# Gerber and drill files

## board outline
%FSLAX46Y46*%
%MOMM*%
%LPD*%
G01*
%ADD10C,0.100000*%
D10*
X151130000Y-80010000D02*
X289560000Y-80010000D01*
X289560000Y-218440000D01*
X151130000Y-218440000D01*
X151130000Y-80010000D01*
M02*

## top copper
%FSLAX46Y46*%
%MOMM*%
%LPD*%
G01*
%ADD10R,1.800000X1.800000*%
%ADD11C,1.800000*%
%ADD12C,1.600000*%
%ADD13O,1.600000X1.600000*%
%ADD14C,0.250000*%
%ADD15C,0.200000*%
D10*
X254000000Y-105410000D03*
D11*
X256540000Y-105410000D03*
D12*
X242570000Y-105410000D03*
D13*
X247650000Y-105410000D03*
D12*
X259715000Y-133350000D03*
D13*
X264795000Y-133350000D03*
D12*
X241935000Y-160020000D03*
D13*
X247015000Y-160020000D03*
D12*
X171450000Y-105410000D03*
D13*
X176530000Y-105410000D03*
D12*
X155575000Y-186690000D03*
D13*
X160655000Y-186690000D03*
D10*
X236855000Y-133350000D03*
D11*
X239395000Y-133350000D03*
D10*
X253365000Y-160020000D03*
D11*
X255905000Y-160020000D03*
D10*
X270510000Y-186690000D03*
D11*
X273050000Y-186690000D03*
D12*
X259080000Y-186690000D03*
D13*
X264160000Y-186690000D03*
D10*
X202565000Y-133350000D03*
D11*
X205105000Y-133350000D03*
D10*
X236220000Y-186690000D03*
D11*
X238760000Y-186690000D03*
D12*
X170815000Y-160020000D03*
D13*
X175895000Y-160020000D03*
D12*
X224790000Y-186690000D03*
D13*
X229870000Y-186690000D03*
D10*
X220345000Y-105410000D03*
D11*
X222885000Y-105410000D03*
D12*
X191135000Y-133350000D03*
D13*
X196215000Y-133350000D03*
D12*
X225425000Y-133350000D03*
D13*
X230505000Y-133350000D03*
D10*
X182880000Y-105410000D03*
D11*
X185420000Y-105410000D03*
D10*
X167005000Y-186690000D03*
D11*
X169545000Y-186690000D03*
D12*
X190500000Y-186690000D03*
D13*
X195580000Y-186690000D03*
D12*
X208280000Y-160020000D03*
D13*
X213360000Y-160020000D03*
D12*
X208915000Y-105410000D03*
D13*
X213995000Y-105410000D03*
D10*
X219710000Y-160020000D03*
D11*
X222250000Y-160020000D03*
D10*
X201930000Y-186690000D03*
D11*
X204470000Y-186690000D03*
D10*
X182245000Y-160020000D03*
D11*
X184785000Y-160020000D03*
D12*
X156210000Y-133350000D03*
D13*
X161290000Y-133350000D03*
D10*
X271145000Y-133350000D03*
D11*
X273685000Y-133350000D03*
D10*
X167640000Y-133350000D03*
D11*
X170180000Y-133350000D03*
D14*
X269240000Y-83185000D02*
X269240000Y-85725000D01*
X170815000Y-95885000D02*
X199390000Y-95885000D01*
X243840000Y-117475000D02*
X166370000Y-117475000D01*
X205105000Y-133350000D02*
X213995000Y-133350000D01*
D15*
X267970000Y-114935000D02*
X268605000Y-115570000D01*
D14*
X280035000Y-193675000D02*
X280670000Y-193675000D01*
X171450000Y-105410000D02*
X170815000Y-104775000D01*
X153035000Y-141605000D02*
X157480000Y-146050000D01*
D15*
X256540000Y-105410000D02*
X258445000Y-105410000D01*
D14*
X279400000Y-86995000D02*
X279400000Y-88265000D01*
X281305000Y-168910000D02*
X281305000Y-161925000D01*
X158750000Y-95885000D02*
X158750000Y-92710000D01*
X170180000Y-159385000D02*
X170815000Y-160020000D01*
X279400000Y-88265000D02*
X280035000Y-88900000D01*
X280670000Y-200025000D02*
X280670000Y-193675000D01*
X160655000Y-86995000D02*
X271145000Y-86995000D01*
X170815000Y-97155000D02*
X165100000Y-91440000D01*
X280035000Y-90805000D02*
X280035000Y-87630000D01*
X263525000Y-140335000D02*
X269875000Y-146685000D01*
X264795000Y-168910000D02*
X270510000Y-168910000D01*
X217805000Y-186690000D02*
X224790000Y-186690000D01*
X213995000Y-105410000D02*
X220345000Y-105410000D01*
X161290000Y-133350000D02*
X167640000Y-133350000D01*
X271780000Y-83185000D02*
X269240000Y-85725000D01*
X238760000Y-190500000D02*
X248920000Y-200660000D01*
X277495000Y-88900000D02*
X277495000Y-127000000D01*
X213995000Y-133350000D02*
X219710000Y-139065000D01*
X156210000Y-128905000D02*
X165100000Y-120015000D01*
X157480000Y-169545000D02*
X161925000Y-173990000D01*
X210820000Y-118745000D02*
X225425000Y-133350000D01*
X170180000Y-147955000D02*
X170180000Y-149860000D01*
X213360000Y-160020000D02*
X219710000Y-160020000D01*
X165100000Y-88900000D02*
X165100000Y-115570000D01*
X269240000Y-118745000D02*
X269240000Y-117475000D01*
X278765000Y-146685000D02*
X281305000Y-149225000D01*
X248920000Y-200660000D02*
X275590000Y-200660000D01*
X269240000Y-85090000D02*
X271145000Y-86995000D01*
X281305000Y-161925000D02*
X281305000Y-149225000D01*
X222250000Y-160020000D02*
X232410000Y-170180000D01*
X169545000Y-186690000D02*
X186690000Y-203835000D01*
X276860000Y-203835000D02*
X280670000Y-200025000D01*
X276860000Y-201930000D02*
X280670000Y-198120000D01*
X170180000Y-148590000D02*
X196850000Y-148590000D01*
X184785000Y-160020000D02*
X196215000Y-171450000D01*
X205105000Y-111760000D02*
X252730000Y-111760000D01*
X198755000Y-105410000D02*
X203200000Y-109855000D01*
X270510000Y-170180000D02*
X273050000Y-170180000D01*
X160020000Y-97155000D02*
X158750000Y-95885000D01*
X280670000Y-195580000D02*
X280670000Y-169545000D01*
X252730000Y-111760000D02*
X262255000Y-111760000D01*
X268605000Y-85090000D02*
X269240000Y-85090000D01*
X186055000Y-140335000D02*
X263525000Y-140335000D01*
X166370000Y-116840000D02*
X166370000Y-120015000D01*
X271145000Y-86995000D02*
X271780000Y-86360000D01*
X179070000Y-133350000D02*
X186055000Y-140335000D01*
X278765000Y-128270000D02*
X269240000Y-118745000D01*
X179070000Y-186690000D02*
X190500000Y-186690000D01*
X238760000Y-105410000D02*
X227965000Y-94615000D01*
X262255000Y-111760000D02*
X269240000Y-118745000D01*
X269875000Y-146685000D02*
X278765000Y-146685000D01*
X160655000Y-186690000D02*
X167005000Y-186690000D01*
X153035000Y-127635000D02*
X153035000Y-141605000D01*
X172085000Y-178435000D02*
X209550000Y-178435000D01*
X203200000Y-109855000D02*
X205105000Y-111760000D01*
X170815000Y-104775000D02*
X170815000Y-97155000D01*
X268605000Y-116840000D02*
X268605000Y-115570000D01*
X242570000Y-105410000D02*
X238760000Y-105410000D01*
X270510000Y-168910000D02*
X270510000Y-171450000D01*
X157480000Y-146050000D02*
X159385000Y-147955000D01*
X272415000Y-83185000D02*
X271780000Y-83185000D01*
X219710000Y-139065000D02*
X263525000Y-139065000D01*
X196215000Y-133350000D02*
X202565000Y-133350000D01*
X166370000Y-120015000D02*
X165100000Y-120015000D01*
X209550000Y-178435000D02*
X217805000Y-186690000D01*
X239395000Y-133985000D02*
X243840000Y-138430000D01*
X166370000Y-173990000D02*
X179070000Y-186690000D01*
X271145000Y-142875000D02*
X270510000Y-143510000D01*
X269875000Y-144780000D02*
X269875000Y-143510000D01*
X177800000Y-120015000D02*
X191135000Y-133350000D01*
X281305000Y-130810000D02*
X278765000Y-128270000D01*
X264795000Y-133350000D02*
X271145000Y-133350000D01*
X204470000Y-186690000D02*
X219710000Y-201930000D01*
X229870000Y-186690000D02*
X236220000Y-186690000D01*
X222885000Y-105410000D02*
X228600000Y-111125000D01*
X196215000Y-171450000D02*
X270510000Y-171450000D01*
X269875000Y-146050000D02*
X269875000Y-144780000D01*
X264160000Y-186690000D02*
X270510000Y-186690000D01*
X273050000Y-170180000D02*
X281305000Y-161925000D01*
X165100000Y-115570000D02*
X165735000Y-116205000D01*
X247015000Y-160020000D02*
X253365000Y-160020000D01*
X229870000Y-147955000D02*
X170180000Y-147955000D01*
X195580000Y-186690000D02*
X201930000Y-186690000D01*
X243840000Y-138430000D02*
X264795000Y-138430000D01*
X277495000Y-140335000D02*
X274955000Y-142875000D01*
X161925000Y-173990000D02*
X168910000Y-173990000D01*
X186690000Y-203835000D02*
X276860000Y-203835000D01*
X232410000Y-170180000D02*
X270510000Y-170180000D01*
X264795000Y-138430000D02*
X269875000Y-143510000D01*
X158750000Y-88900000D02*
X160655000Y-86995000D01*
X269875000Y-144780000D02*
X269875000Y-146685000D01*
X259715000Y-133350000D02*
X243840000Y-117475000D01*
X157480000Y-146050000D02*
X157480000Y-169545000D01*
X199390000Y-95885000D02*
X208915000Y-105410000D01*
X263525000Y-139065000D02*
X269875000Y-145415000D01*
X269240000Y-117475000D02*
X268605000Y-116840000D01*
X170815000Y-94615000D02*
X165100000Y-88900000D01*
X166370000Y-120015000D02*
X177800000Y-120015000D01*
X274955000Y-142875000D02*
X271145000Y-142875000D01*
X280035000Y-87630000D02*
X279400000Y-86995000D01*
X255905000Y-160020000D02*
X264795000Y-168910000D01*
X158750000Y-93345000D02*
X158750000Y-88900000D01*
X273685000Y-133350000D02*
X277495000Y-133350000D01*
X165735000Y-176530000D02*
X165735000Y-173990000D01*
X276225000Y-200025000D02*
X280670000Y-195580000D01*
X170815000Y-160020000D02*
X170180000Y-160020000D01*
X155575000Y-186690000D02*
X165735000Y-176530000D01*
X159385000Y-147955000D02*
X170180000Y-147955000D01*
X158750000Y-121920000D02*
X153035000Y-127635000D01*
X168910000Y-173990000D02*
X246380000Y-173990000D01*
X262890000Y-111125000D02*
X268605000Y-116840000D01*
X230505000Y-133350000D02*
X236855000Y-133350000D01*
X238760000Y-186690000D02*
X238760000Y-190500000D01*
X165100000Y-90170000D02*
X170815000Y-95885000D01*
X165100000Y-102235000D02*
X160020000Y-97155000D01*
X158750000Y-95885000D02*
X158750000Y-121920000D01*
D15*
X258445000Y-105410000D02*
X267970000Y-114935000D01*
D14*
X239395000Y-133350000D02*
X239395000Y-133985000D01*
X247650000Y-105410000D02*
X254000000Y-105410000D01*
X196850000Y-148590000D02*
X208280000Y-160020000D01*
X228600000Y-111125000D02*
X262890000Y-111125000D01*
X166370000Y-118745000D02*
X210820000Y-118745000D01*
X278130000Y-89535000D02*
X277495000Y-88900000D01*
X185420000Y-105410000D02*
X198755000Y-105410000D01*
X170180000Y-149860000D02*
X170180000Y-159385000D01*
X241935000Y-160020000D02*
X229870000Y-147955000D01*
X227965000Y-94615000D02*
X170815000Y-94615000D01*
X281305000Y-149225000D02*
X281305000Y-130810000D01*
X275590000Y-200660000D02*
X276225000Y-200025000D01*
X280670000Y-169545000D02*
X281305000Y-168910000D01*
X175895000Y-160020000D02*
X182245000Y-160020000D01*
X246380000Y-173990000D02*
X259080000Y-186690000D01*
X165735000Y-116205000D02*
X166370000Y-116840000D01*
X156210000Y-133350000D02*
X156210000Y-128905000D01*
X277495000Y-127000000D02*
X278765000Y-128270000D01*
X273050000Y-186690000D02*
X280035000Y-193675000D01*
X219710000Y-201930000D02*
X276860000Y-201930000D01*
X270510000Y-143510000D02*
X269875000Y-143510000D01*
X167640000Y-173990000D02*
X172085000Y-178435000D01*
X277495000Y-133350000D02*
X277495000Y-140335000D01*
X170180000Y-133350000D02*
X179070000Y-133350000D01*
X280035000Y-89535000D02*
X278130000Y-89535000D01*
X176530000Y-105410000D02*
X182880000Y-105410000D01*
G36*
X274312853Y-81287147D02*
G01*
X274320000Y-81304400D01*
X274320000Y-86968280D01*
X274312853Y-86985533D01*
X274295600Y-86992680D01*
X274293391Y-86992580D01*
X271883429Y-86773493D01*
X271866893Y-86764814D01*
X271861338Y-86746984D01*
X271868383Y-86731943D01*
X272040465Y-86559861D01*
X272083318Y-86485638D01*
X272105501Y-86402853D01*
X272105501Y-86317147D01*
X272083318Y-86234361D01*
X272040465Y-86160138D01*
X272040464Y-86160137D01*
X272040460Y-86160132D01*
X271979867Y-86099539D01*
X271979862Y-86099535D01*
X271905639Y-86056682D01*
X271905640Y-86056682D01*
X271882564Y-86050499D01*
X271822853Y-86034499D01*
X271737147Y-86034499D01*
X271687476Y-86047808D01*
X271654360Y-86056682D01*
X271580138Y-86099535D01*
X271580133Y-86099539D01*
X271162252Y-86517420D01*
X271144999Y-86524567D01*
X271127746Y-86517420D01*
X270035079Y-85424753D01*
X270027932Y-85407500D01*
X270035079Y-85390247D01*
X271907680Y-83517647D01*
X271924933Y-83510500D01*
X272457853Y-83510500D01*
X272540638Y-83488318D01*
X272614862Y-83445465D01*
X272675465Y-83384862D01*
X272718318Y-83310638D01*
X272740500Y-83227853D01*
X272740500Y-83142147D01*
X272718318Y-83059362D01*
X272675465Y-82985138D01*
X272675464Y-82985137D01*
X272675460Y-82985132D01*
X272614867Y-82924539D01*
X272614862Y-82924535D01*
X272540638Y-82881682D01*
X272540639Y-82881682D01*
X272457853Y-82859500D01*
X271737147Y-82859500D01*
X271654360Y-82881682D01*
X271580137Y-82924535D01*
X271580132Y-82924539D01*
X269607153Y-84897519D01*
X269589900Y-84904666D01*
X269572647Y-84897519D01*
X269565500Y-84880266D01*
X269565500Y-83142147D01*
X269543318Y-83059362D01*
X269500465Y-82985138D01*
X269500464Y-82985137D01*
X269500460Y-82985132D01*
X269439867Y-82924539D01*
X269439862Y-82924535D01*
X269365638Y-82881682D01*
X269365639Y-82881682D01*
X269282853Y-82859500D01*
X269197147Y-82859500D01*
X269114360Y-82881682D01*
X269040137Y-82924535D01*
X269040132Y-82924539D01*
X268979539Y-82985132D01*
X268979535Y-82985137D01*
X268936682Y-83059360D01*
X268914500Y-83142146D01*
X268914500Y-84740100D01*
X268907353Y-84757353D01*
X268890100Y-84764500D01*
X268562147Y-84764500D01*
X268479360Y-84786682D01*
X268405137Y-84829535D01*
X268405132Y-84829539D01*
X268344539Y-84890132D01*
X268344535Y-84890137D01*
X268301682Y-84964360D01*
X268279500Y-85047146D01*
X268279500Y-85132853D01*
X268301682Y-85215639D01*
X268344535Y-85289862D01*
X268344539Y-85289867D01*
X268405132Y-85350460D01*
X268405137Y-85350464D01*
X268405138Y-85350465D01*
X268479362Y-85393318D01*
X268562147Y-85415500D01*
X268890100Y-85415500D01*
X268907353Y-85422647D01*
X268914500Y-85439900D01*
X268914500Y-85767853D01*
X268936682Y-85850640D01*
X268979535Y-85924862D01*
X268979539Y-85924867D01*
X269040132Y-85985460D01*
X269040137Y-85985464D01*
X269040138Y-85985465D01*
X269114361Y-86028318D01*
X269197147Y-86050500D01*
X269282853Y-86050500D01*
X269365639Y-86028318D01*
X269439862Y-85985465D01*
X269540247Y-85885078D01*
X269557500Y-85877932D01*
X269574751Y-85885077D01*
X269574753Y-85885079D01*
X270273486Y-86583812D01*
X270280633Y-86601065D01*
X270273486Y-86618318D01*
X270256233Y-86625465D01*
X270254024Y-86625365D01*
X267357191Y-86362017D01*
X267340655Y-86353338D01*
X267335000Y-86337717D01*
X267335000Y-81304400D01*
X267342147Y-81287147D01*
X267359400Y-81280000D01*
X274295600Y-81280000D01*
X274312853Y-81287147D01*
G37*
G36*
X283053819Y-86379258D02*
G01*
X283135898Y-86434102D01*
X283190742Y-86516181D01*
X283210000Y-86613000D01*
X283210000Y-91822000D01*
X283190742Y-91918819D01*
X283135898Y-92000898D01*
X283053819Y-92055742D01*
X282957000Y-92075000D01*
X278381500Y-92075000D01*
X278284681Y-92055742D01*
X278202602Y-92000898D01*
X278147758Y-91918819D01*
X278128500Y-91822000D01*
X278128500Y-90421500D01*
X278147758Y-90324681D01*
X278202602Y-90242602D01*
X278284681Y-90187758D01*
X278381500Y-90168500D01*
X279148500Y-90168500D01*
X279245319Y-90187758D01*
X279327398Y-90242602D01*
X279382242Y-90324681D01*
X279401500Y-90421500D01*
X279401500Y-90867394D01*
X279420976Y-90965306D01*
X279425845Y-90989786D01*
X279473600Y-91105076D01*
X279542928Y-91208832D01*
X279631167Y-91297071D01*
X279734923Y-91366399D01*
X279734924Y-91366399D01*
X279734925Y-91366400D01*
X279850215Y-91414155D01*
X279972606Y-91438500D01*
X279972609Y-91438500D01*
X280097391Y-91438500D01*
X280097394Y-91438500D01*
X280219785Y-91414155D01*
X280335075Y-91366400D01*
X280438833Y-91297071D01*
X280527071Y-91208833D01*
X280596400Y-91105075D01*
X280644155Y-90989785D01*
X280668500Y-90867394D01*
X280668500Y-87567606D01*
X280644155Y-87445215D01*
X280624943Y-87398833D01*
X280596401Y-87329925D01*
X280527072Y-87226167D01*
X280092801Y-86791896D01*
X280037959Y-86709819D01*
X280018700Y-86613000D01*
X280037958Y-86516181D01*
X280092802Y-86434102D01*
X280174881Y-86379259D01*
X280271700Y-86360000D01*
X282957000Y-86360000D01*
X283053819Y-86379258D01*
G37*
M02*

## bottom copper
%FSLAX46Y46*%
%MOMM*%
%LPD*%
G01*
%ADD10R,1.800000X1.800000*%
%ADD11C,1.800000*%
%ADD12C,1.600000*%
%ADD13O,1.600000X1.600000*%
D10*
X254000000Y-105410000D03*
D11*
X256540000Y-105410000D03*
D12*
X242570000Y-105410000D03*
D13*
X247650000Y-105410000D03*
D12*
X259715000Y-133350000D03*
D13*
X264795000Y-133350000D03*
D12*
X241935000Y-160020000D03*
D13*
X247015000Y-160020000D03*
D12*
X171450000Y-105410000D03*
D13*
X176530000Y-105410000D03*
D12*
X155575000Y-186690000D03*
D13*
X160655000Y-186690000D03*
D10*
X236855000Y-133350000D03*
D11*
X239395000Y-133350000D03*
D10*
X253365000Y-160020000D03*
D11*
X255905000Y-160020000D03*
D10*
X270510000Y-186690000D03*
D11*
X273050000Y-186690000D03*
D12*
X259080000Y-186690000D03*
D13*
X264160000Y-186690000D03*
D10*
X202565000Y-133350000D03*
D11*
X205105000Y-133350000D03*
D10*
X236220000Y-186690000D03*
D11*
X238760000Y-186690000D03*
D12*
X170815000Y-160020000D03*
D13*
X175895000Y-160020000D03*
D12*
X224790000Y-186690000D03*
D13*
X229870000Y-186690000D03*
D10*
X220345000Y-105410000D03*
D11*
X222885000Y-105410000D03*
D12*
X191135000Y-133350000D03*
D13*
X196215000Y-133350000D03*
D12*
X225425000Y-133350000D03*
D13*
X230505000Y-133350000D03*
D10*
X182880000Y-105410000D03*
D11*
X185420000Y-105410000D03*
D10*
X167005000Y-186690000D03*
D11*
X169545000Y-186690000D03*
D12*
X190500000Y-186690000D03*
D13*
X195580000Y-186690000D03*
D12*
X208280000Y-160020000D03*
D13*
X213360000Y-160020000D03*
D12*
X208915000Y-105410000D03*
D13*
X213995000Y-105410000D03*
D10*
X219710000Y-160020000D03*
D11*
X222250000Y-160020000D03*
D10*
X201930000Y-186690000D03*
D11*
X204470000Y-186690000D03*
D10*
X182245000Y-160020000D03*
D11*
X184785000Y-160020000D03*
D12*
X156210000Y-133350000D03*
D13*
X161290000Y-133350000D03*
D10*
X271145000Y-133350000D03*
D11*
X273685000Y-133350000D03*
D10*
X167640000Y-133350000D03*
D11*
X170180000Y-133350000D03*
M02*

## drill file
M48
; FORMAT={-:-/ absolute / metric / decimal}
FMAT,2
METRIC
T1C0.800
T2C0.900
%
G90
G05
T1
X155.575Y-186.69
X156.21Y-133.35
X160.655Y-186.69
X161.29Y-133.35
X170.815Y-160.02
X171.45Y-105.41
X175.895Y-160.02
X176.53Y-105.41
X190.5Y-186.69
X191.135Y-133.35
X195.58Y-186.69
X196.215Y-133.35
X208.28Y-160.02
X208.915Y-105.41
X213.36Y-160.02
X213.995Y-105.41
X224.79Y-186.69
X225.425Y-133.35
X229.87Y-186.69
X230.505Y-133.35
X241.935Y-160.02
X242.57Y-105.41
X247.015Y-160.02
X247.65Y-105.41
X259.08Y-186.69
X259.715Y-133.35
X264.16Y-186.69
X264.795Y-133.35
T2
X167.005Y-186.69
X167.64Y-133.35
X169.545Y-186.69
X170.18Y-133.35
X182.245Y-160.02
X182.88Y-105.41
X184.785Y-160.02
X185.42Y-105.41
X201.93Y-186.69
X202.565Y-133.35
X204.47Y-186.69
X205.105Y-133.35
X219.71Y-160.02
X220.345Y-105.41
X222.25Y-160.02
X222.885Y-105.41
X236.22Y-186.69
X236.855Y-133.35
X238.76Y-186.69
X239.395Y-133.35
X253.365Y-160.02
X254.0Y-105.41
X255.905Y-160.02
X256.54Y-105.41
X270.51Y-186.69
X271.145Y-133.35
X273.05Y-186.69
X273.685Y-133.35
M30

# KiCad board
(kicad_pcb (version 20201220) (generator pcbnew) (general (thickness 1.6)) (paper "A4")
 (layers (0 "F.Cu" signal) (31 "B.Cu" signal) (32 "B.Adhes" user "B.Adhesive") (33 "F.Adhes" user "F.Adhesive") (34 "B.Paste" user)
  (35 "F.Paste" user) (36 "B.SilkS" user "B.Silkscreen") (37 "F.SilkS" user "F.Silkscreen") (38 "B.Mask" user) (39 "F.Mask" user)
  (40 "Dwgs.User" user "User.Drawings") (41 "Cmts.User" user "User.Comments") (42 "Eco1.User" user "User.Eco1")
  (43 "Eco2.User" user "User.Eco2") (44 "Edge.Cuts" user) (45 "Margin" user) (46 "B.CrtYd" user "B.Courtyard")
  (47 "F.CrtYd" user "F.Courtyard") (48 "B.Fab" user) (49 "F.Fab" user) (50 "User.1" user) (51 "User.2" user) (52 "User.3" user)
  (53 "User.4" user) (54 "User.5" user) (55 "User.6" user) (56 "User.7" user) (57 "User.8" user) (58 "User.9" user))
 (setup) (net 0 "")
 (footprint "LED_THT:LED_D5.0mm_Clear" (layer "F.Cu") (at 254 105.41)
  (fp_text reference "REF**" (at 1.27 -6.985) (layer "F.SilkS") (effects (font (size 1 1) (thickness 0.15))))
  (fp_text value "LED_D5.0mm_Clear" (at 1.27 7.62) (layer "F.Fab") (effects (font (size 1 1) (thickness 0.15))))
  (pad "1" thru_hole rect (at 0 0) (size 1.8 1.8) (drill 0.9) (layers *.Cu *.Mask))
  (pad "2" thru_hole circle (at 2.54 0) (size 1.8 1.8) (drill 0.9) (layers *.Cu *.Mask)))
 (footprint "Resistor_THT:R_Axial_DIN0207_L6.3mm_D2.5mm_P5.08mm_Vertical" (layer "F.Cu") (at 242.57 105.41)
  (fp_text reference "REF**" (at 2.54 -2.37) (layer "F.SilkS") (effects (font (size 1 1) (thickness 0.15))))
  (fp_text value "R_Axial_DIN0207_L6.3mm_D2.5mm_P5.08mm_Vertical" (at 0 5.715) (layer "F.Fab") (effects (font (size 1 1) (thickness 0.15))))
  (pad "1" thru_hole circle (at 0 0) (size 1.6 1.6) (drill 0.8) (layers *.Cu *.Mask))
  (pad "2" thru_hole oval (at 5.08 0) (size 1.6 1.6) (drill 0.8) (layers *.Cu *.Mask)))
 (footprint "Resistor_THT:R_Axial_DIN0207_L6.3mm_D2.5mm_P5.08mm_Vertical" (layer "F.Cu") (at 259.715 133.35)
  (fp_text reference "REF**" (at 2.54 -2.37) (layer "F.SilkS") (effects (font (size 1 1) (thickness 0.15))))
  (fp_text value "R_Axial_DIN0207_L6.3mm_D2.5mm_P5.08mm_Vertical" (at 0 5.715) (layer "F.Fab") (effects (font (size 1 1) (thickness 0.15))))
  (pad "1" thru_hole circle (at 0 0) (size 1.6 1.6) (drill 0.8) (layers *.Cu *.Mask))
  (pad "2" thru_hole oval (at 5.08 0) (size 1.6 1.6) (drill 0.8) (layers *.Cu *.Mask)))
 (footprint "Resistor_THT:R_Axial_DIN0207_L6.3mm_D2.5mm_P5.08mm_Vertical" (layer "F.Cu") (at 241.935 160.02)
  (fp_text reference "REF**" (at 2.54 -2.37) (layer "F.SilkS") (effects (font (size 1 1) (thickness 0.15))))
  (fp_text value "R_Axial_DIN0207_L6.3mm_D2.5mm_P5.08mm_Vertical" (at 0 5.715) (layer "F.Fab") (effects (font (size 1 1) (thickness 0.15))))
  (pad "1" thru_hole circle (at 0 0) (size 1.6 1.6) (drill 0.8) (layers *.Cu *.Mask))
  (pad "2" thru_hole oval (at 5.08 0) (size 1.6 1.6) (drill 0.8) (layers *.Cu *.Mask)))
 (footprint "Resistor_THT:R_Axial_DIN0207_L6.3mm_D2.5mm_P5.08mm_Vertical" (layer "F.Cu") (at 171.45 105.41)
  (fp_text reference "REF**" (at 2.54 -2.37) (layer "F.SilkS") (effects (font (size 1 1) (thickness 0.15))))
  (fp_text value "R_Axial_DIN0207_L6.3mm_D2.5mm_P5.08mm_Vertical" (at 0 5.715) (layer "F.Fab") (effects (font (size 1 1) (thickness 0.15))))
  (pad "1" thru_hole circle (at 0 0) (size 1.6 1.6) (drill 0.8) (layers *.Cu *.Mask))
  (pad "2" thru_hole oval (at 5.08 0) (size 1.6 1.6) (drill 0.8) (layers *.Cu *.Mask)))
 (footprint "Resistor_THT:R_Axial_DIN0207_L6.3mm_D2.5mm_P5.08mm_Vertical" (layer "F.Cu") (at 155.575 186.69)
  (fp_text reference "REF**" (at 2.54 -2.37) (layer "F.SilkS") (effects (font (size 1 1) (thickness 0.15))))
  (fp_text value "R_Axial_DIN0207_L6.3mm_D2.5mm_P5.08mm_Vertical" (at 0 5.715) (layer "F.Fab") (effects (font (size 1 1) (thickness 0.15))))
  (pad "1" thru_hole circle (at 0 0) (size 1.6 1.6) (drill 0.8) (layers *.Cu *.Mask))
  (pad "2" thru_hole oval (at 5.08 0) (size 1.6 1.6) (drill 0.8) (layers *.Cu *.Mask)))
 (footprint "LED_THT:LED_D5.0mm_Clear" (layer "F.Cu") (at 236.855 133.35)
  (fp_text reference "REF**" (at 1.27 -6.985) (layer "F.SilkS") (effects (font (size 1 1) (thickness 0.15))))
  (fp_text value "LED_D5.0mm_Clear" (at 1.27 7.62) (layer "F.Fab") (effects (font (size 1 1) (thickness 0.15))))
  (pad "1" thru_hole rect (at 0 0) (size 1.8 1.8) (drill 0.9) (layers *.Cu *.Mask))
  (pad "2" thru_hole circle (at 2.54 0) (size 1.8 1.8) (drill 0.9) (layers *.Cu *.Mask)))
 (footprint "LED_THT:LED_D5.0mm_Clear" (layer "F.Cu") (at 253.365 160.02)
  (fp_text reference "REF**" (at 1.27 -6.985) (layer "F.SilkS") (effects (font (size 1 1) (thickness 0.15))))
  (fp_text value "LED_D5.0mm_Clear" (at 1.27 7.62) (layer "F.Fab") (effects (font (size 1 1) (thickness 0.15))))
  (pad "1" thru_hole rect (at 0 0) (size 1.8 1.8) (drill 0.9) (layers *.Cu *.Mask))
  (pad "2" thru_hole circle (at 2.54 0) (size 1.8 1.8) (drill 0.9) (layers *.Cu *.Mask)))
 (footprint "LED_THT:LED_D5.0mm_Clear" (layer "F.Cu") (at 270.51 186.69)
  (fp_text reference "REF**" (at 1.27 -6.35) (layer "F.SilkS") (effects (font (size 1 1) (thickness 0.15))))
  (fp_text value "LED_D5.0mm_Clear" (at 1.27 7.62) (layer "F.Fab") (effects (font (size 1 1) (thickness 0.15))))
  (pad "1" thru_hole rect (at 0 0) (size 1.8 1.8) (drill 0.9) (layers *.Cu *.Mask))
  (pad "2" thru_hole circle (at 2.54 0) (size 1.8 1.8) (drill 0.9) (layers *.Cu *.Mask)))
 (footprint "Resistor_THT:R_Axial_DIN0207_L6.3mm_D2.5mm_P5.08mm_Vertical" (layer "F.Cu") (at 259.08 186.69)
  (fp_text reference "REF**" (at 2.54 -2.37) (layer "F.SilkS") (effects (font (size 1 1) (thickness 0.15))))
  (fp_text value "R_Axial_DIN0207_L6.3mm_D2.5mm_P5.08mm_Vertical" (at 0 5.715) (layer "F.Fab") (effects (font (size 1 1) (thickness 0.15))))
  (pad "1" thru_hole circle (at 0 0) (size 1.6 1.6) (drill 0.8) (layers *.Cu *.Mask))
  (pad "2" thru_hole oval (at 5.08 0) (size 1.6 1.6) (drill 0.8) (layers *.Cu *.Mask)))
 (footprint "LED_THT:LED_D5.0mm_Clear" (layer "F.Cu") (at 202.565 133.35)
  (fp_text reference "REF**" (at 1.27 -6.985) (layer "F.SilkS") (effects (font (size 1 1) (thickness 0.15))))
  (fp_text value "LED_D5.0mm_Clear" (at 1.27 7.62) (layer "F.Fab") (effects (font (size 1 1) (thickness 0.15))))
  (pad "1" thru_hole rect (at 0 0) (size 1.8 1.8) (drill 0.9) (layers *.Cu *.Mask))
  (pad "2" thru_hole circle (at 2.54 0) (size 1.8 1.8) (drill 0.9) (layers *.Cu *.Mask)))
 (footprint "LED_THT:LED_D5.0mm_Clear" (layer "F.Cu") (at 236.22 186.69)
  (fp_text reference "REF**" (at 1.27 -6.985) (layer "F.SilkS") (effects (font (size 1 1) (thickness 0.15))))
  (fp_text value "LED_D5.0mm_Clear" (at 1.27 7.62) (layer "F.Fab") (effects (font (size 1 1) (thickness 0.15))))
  (pad "1" thru_hole rect (at 0 0) (size 1.8 1.8) (drill 0.9) (layers *.Cu *.Mask))
  (pad "2" thru_hole circle (at 2.54 0) (size 1.8 1.8) (drill 0.9) (layers *.Cu *.Mask)))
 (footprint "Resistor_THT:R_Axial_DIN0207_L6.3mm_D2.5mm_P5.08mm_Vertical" (layer "F.Cu") (at 170.815 160.02)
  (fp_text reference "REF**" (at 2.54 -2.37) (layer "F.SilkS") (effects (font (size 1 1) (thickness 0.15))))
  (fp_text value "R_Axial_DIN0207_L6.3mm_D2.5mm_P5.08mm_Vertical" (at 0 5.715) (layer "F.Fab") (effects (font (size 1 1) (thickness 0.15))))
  (pad "1" thru_hole circle (at 0 0) (size 1.6 1.6) (drill 0.8) (layers *.Cu *.Mask))
  (pad "2" thru_hole oval (at 5.08 0) (size 1.6 1.6) (drill 0.8) (layers *.Cu *.Mask)))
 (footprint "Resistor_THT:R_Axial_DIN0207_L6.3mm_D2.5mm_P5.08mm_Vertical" (layer "F.Cu") (at 224.79 186.69)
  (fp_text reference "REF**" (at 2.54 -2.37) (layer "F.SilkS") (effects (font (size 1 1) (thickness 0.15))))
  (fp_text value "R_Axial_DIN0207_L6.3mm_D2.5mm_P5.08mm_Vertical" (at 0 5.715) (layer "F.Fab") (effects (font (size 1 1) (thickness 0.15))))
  (pad "1" thru_hole circle (at 0 0) (size 1.6 1.6) (drill 0.8) (layers *.Cu *.Mask))
  (pad "2" thru_hole oval (at 5.08 0) (size 1.6 1.6) (drill 0.8) (layers *.Cu *.Mask)))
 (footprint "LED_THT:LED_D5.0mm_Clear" (layer "F.Cu") (at 220.345 105.41)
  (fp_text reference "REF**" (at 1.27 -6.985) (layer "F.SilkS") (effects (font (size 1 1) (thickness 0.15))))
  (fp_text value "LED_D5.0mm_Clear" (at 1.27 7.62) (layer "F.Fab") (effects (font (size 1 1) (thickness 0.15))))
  (pad "1" thru_hole rect (at 0 0) (size 1.8 1.8) (drill 0.9) (layers *.Cu *.Mask))
  (pad "2" thru_hole circle (at 2.54 0) (size 1.8 1.8) (drill 0.9) (layers *.Cu *.Mask)))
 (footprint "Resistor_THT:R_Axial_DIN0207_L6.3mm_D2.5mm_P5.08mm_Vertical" (layer "F.Cu") (at 191.135 133.35)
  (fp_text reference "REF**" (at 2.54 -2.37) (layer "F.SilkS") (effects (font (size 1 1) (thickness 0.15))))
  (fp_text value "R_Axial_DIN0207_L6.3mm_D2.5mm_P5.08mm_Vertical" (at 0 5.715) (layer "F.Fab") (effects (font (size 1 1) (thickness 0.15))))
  (pad "1" thru_hole circle (at 0 0) (size 1.6 1.6) (drill 0.8) (layers *.Cu *.Mask))
  (pad "2" thru_hole oval (at 5.08 0) (size 1.6 1.6) (drill 0.8) (layers *.Cu *.Mask)))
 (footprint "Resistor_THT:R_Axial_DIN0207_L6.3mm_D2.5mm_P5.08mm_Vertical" (layer "F.Cu") (at 225.425 133.35)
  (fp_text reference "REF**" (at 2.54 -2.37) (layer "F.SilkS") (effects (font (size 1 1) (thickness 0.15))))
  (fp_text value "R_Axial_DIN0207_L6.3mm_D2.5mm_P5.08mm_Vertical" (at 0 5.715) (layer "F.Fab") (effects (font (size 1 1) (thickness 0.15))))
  (pad "1" thru_hole circle (at 0 0) (size 1.6 1.6) (drill 0.8) (layers *.Cu *.Mask))
  (pad "2" thru_hole oval (at 5.08 0) (size 1.6 1.6) (drill 0.8) (layers *.Cu *.Mask)))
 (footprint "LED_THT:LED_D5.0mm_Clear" (layer "F.Cu") (at 182.88 105.41)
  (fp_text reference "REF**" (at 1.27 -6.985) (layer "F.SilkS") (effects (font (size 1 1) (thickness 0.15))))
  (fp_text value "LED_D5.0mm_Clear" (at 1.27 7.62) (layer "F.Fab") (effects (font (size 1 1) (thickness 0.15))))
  (pad "1" thru_hole rect (at 0 0) (size 1.8 1.8) (drill 0.9) (layers *.Cu *.Mask))
  (pad "2" thru_hole circle (at 2.54 0) (size 1.8 1.8) (drill 0.9) (layers *.Cu *.Mask)))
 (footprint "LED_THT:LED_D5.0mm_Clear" (layer "F.Cu") (at 167.005 186.69)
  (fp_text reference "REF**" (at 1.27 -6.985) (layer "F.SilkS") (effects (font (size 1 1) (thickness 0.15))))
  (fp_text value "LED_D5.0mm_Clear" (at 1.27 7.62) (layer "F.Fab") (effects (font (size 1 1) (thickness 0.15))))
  (pad "1" thru_hole rect (at 0 0) (size 1.8 1.8) (drill 0.9) (layers *.Cu *.Mask))
  (pad "2" thru_hole circle (at 2.54 0) (size 1.8 1.8) (drill 0.9) (layers *.Cu *.Mask)))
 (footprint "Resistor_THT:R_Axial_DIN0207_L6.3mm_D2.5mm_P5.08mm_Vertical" (layer "F.Cu") (at 190.5 186.69)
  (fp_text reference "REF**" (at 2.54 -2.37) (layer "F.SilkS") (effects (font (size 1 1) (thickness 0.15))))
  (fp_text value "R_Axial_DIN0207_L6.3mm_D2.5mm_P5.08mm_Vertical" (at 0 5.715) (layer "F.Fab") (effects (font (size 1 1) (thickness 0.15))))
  (pad "1" thru_hole circle (at 0 0) (size 1.6 1.6) (drill 0.8) (layers *.Cu *.Mask))
  (pad "2" thru_hole oval (at 5.08 0) (size 1.6 1.6) (drill 0.8) (layers *.Cu *.Mask)))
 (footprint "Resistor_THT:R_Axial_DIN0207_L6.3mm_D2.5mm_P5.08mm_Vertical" (layer "F.Cu") (at 208.28 160.02)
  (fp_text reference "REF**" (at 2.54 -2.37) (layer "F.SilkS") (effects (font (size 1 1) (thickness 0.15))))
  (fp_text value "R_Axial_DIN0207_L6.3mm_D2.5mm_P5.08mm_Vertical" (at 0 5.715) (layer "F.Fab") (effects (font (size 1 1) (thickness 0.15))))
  (pad "1" thru_hole circle (at 0 0) (size 1.6 1.6) (drill 0.8) (layers *.Cu *.Mask))
  (pad "2" thru_hole oval (at 5.08 0) (size 1.6 1.6) (drill 0.8) (layers *.Cu *.Mask)))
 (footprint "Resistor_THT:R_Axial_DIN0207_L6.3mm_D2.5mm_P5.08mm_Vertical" (layer "F.Cu") (at 208.915 105.41)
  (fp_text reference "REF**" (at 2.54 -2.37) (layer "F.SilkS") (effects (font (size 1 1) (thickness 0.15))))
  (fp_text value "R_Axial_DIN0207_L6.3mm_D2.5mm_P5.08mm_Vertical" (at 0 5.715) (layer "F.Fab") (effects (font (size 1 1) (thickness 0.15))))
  (pad "1" thru_hole circle (at 0 0) (size 1.6 1.6) (drill 0.8) (layers *.Cu *.Mask))
  (pad "2" thru_hole oval (at 5.08 0) (size 1.6 1.6) (drill 0.8) (layers *.Cu *.Mask)))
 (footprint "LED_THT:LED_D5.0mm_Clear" (layer "F.Cu") (at 219.71 160.02)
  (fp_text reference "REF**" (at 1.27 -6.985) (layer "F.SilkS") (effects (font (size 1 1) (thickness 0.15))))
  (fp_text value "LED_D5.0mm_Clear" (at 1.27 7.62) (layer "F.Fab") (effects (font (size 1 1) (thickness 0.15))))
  (pad "1" thru_hole rect (at 0 0) (size 1.8 1.8) (drill 0.9) (layers *.Cu *.Mask))
  (pad "2" thru_hole circle (at 2.54 0) (size 1.8 1.8) (drill 0.9) (layers *.Cu *.Mask)))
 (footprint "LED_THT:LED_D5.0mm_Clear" (layer "F.Cu") (at 201.93 186.69)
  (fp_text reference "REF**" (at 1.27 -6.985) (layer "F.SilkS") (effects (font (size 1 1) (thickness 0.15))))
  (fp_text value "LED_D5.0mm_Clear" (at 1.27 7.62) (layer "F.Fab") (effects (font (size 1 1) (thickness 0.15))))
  (pad "1" thru_hole rect (at 0 0) (size 1.8 1.8) (drill 0.9) (layers *.Cu *.Mask))
  (pad "2" thru_hole circle (at 2.54 0) (size 1.8 1.8) (drill 0.9) (layers *.Cu *.Mask)))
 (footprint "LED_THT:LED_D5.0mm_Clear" (layer "F.Cu") (at 182.245 160.02)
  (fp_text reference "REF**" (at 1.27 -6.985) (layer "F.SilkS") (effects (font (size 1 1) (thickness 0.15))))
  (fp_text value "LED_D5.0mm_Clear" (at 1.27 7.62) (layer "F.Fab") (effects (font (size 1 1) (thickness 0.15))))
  (pad "1" thru_hole rect (at 0 0) (size 1.8 1.8) (drill 0.9) (layers *.Cu *.Mask))
  (pad "2" thru_hole circle (at 2.54 0) (size 1.8 1.8) (drill 0.9) (layers *.Cu *.Mask)))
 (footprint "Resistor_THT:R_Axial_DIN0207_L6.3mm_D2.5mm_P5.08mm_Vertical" (layer "F.Cu") (at 156.21 133.35)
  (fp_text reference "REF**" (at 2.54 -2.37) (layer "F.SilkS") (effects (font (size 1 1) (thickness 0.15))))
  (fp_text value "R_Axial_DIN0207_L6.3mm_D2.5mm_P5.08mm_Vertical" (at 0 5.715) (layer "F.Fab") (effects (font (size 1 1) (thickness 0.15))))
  (pad "1" thru_hole circle (at 0 0) (size 1.6 1.6) (drill 0.8) (layers *.Cu *.Mask))
  (pad "2" thru_hole oval (at 5.08 0) (size 1.6 1.6) (drill 0.8) (layers *.Cu *.Mask)))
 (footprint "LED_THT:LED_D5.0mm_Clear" (layer "F.Cu") (at 271.145 133.35)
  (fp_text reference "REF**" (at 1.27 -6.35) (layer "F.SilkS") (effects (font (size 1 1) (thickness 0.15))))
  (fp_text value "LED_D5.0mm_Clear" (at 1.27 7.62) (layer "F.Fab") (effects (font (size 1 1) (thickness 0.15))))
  (pad "1" thru_hole rect (at 0 0) (size 1.8 1.8) (drill 0.9) (layers *.Cu *.Mask))
  (pad "2" thru_hole circle (at 2.54 0) (size 1.8 1.8) (drill 0.9) (layers *.Cu *.Mask)))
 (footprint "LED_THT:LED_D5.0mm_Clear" (layer "F.Cu") (at 167.64 133.35)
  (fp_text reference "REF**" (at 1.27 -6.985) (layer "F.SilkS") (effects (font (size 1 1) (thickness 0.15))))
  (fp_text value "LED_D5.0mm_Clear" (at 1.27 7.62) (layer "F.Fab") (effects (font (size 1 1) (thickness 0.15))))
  (pad "1" thru_hole rect (at 0 0) (size 1.8 1.8) (drill 0.9) (layers *.Cu *.Mask))
  (pad "2" thru_hole circle (at 2.54 0) (size 1.8 1.8) (drill 0.9) (layers *.Cu *.Mask)))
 (gr_rect (start 151.13 80.01) (end 289.56 218.44) (layer "Edge.Cuts") (width 0.1) (fill none))
 (segment (start 269.24 83.185) (end 269.24 85.725) (width 0.25) (layer "F.Cu") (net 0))
 (segment (start 170.815 95.885) (end 199.39 95.885) (width 0.25) (layer "F.Cu") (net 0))
 (segment (start 243.84 117.475) (end 166.37 117.475) (width 0.25) (layer "F.Cu") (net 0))
 (segment (start 205.105 133.35) (end 213.995 133.35) (width 0.25) (layer "F.Cu") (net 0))
 (segment (start 267.97 114.935) (end 268.605 115.57) (width 0.2) (layer "F.Cu") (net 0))
 (segment (start 280.035 193.675) (end 280.67 193.675) (width 0.25) (layer "F.Cu") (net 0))
 (segment (start 171.45 105.41) (end 170.815 104.775) (width 0.25) (layer "F.Cu") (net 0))
 (segment (start 153.035 141.605) (end 157.48 146.05) (width 0.25) (layer "F.Cu") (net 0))
 (segment (start 256.54 105.41) (end 258.445 105.41) (width 0.2) (layer "F.Cu") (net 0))
 (segment (start 279.4 86.995) (end 279.4 88.265) (width 0.25) (layer "F.Cu") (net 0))
 (segment (start 281.305 168.91) (end 281.305 161.925) (width 0.25) (layer "F.Cu") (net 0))
 (segment (start 158.75 95.885) (end 158.75 92.71) (width 0.25) (layer "F.Cu") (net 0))
 (segment (start 170.18 159.385) (end 170.815 160.02) (width 0.25) (layer "F.Cu") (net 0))
 (segment (start 279.4 88.265) (end 280.035 88.9) (width 0.25) (layer "F.Cu") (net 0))
 (segment (start 280.67 200.025) (end 280.67 193.675) (width 0.25) (layer "F.Cu") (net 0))
 (segment (start 160.655 86.995) (end 271.145 86.995) (width 0.25) (layer "F.Cu") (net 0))
 (segment (start 170.815 97.155) (end 165.1 91.44) (width 0.25) (layer "F.Cu") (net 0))
 (segment (start 280.035 90.805) (end 280.035 87.63) (width 0.25) (layer "F.Cu") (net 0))
 (segment (start 263.525 140.335) (end 269.875 146.685) (width 0.25) (layer "F.Cu") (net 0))
 (segment (start 264.795 168.91) (end 270.51 168.91) (width 0.25) (layer "F.Cu") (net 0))
 (segment (start 217.805 186.69) (end 224.79 186.69) (width 0.25) (layer "F.Cu") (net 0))
 (segment (start 213.995 105.41) (end 220.345 105.41) (width 0.25) (layer "F.Cu") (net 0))
 (segment (start 161.29 133.35) (end 167.64 133.35) (width 0.25) (layer "F.Cu") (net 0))
 (segment (start 271.78 83.185) (end 269.24 85.725) (width 0.25) (layer "F.Cu") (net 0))
 (segment (start 238.76 190.5) (end 248.92 200.66) (width 0.25) (layer "F.Cu") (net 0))
 (segment (start 277.495 88.9) (end 277.495 127) (width 0.25) (layer "F.Cu") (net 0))
 (segment (start 213.995 133.35) (end 219.71 139.065) (width 0.25) (layer "F.Cu") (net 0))
 (segment (start 156.21 128.905) (end 165.1 120.015) (width 0.25) (layer "F.Cu") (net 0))
 (segment (start 157.48 169.545) (end 161.925 173.99) (width 0.25) (layer "F.Cu") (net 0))
 (segment (start 210.82 118.745) (end 225.425 133.35) (width 0.25) (layer "F.Cu") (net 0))
 (segment (start 170.18 147.955) (end 170.18 149.86) (width 0.25) (layer "F.Cu") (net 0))
 (segment (start 213.36 160.02) (end 219.71 160.02) (width 0.25) (layer "F.Cu") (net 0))
 (segment (start 165.1 88.9) (end 165.1 115.57) (width 0.25) (layer "F.Cu") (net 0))
 (segment (start 269.24 118.745) (end 269.24 117.475) (width 0.25) (layer "F.Cu") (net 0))
 (segment (start 278.765 146.685) (end 281.305 149.225) (width 0.25) (layer "F.Cu") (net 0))
 (segment (start 248.92 200.66) (end 275.59 200.66) (width 0.25) (layer "F.Cu") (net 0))
 (segment (start 269.24 85.09) (end 271.145 86.995) (width 0.25) (layer "F.Cu") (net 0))
 (segment (start 281.305 161.925) (end 281.305 149.225) (width 0.25) (layer "F.Cu") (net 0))
 (segment (start 222.25 160.02) (end 232.41 170.18) (width 0.25) (layer "F.Cu") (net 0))
 (segment (start 169.545 186.69) (end 186.69 203.835) (width 0.25) (layer "F.Cu") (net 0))
 (segment (start 276.86 203.835) (end 280.67 200.025) (width 0.25) (layer "F.Cu") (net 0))
 (segment (start 276.86 201.93) (end 280.67 198.12) (width 0.25) (layer "F.Cu") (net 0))
 (segment (start 170.18 148.59) (end 196.85 148.59) (width 0.25) (layer "F.Cu") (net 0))
 (segment (start 184.785 160.02) (end 196.215 171.45) (width 0.25) (layer "F.Cu") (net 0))
 (segment (start 205.105 111.76) (end 252.73 111.76) (width 0.25) (layer "F.Cu") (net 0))
 (segment (start 198.755 105.41) (end 203.2 109.855) (width 0.25) (layer "F.Cu") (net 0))
 (segment (start 270.51 170.18) (end 273.05 170.18) (width 0.25) (layer "F.Cu") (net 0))
 (segment (start 160.02 97.155) (end 158.75 95.885) (width 0.25) (layer "F.Cu") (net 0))
 (segment (start 280.67 195.58) (end 280.67 169.545) (width 0.25) (layer "F.Cu") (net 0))
 (segment (start 252.73 111.76) (end 262.255 111.76) (width 0.25) (layer "F.Cu") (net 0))
 (segment (start 268.605 85.09) (end 269.24 85.09) (width 0.25) (layer "F.Cu") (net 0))
 (segment (start 186.055 140.335) (end 263.525 140.335) (width 0.25) (layer "F.Cu") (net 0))
 (segment (start 166.37 116.84) (end 166.37 120.015) (width 0.25) (layer "F.Cu") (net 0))
 (segment (start 271.145 86.995) (end 271.78 86.36) (width 0.25) (layer "F.Cu") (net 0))
 (segment (start 179.07 133.35) (end 186.055 140.335) (width 0.25) (layer "F.Cu") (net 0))
 (segment (start 278.765 128.27) (end 269.24 118.745) (width 0.25) (layer "F.Cu") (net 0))
 (segment (start 179.07 186.69) (end 190.5 186.69) (width 0.25) (layer "F.Cu") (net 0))
 (segment (start 238.76 105.41) (end 227.965 94.615) (width 0.25) (layer "F.Cu") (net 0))
 (segment (start 262.255 111.76) (end 269.24 118.745) (width 0.25) (layer "F.Cu") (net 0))
 (segment (start 269.875 146.685) (end 278.765 146.685) (width 0.25) (layer "F.Cu") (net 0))
 (segment (start 160.655 186.69) (end 167.005 186.69) (width 0.25) (layer "F.Cu") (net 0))
 (segment (start 153.035 127.635) (end 153.035 141.605) (width 0.25) (layer "F.Cu") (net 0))
 (segment (start 172.085 178.435) (end 209.55 178.435) (width 0.25) (layer "F.Cu") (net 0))
 (segment (start 203.2 109.855) (end 205.105 111.76) (width 0.25) (layer "F.Cu") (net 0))
 (segment (start 170.815 104.775) (end 170.815 97.155) (width 0.25) (layer "F.Cu") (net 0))
 (segment (start 268.605 116.84) (end 268.605 115.57) (width 0.25) (layer "F.Cu") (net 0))
 (segment (start 242.57 105.41) (end 238.76 105.41) (width 0.25) (layer "F.Cu") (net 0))
 (segment (start 270.51 168.91) (end 270.51 171.45) (width 0.25) (layer "F.Cu") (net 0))
 (segment (start 157.48 146.05) (end 159.385 147.955) (width 0.25) (layer "F.Cu") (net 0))
 (segment (start 272.415 83.185) (end 271.78 83.185) (width 0.25) (layer "F.Cu") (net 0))
 (segment (start 219.71 139.065) (end 263.525 139.065) (width 0.25) (layer "F.Cu") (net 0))
 (segment (start 196.215 133.35) (end 202.565 133.35) (width 0.25) (layer "F.Cu") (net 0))
 (segment (start 166.37 120.015) (end 165.1 120.015) (width 0.25) (layer "F.Cu") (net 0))
 (segment (start 209.55 178.435) (end 217.805 186.69) (width 0.25) (layer "F.Cu") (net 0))
 (segment (start 239.395 133.985) (end 243.84 138.43) (width 0.25) (layer "F.Cu") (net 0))
 (segment (start 166.37 173.99) (end 179.07 186.69) (width 0.25) (layer "F.Cu") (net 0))
 (segment (start 271.145 142.875) (end 270.51 143.51) (width 0.25) (layer "F.Cu") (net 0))
 (segment (start 269.875 144.78) (end 269.875 143.51) (width 0.25) (layer "F.Cu") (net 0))
 (segment (start 177.8 120.015) (end 191.135 133.35) (width 0.25) (layer "F.Cu") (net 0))
 (segment (start 281.305 130.81) (end 278.765 128.27) (width 0.25) (layer "F.Cu") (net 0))
 (segment (start 264.795 133.35) (end 271.145 133.35) (width 0.25) (layer "F.Cu") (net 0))
 (segment (start 204.47 186.69) (end 219.71 201.93) (width 0.25) (layer "F.Cu") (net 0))
 (segment (start 229.87 186.69) (end 236.22 186.69) (width 0.25) (layer "F.Cu") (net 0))
 (segment (start 222.885 105.41) (end 228.6 111.125) (width 0.25) (layer "F.Cu") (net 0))
 (segment (start 196.215 171.45) (end 270.51 171.45) (width 0.25) (layer "F.Cu") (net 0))
 (segment (start 269.875 146.05) (end 269.875 144.78) (width 0.25) (layer "F.Cu") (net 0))
 (segment (start 264.16 186.69) (end 270.51 186.69) (width 0.25) (layer "F.Cu") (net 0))
 (segment (start 273.05 170.18) (end 281.305 161.925) (width 0.25) (layer "F.Cu") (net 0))
 (segment (start 165.1 115.57) (end 165.735 116.205) (width 0.25) (layer "F.Cu") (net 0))
 (segment (start 247.015 160.02) (end 253.365 160.02) (width 0.25) (layer "F.Cu") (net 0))
 (segment (start 229.87 147.955) (end 170.18 147.955) (width 0.25) (layer "F.Cu") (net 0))
 (segment (start 195.58 186.69) (end 201.93 186.69) (width 0.25) (layer "F.Cu") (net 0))
 (segment (start 243.84 138.43) (end 264.795 138.43) (width 0.25) (layer "F.Cu") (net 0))
 (segment (start 277.495 140.335) (end 274.955 142.875) (width 0.25) (layer "F.Cu") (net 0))
 (segment (start 161.925 173.99) (end 168.91 173.99) (width 0.25) (layer "F.Cu") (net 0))
 (segment (start 186.69 203.835) (end 276.86 203.835) (width 0.25) (layer "F.Cu") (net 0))
 (segment (start 232.41 170.18) (end 270.51 170.18) (width 0.25) (layer "F.Cu") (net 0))
 (segment (start 264.795 138.43) (end 269.875 143.51) (width 0.25) (layer "F.Cu") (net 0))
 (segment (start 158.75 88.9) (end 160.655 86.995) (width 0.25) (layer "F.Cu") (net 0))
 (segment (start 269.875 144.78) (end 269.875 146.685) (width 0.25) (layer "F.Cu") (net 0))
 (segment (start 259.715 133.35) (end 243.84 117.475) (width 0.25) (layer "F.Cu") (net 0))
 (segment (start 157.48 146.05) (end 157.48 169.545) (width 0.25) (layer "F.Cu") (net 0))
 (segment (start 199.39 95.885) (end 208.915 105.41) (width 0.25) (layer "F.Cu") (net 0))
 (segment (start 263.525 139.065) (end 269.875 145.415) (width 0.25) (layer "F.Cu") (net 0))
 (segment (start 269.24 117.475) (end 268.605 116.84) (width 0.25) (layer "F.Cu") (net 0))
 (segment (start 170.815 94.615) (end 165.1 88.9) (width 0.25) (layer "F.Cu") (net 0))
 (segment (start 166.37 120.015) (end 177.8 120.015) (width 0.25) (layer "F.Cu") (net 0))
 (segment (start 274.955 142.875) (end 271.145 142.875) (width 0.25) (layer "F.Cu") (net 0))
 (segment (start 280.035 87.63) (end 279.4 86.995) (width 0.25) (layer "F.Cu") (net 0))
 (segment (start 255.905 160.02) (end 264.795 168.91) (width 0.25) (layer "F.Cu") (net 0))
 (segment (start 158.75 93.345) (end 158.75 88.9) (width 0.25) (layer "F.Cu") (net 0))
 (segment (start 273.685 133.35) (end 277.495 133.35) (width 0.25) (layer "F.Cu") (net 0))
 (segment (start 165.735 176.53) (end 165.735 173.99) (width 0.25) (layer "F.Cu") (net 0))
 (segment (start 276.225 200.025) (end 280.67 195.58) (width 0.25) (layer "F.Cu") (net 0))
 (segment (start 170.815 160.02) (end 170.18 160.02) (width 0.25) (layer "F.Cu") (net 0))
 (segment (start 155.575 186.69) (end 165.735 176.53) (width 0.25) (layer "F.Cu") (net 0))
 (segment (start 159.385 147.955) (end 170.18 147.955) (width 0.25) (layer "F.Cu") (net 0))
 (segment (start 158.75 121.92) (end 153.035 127.635) (width 0.25) (layer "F.Cu") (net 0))
 (segment (start 168.91 173.99) (end 246.38 173.99) (width 0.25) (layer "F.Cu") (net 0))
 (segment (start 262.89 111.125) (end 268.605 116.84) (width 0.25) (layer "F.Cu") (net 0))
 (segment (start 230.505 133.35) (end 236.855 133.35) (width 0.25) (layer "F.Cu") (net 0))
 (segment (start 238.76 186.69) (end 238.76 190.5) (width 0.25) (layer "F.Cu") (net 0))
 (segment (start 165.1 90.17) (end 170.815 95.885) (width 0.25) (layer "F.Cu") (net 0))
 (segment (start 165.1 102.235) (end 160.02 97.155) (width 0.25) (layer "F.Cu") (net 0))
 (segment (start 158.75 95.885) (end 158.75 121.92) (width 0.25) (layer "F.Cu") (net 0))
 (segment (start 258.445 105.41) (end 267.97 114.935) (width 0.2) (layer "F.Cu") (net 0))
 (segment (start 239.395 133.35) (end 239.395 133.985) (width 0.25) (layer "F.Cu") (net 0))
 (segment (start 247.65 105.41) (end 254 105.41) (width 0.25) (layer "F.Cu") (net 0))
 (segment (start 196.85 148.59) (end 208.28 160.02) (width 0.25) (layer "F.Cu") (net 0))
 (segment (start 228.6 111.125) (end 262.89 111.125) (width 0.25) (layer "F.Cu") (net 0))
 (segment (start 166.37 118.745) (end 210.82 118.745) (width 0.25) (layer "F.Cu") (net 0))
 (segment (start 278.13 89.535) (end 277.495 88.9) (width 0.25) (layer "F.Cu") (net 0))
 (segment (start 185.42 105.41) (end 198.755 105.41) (width 0.25) (layer "F.Cu") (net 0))
 (segment (start 170.18 149.86) (end 170.18 159.385) (width 0.25) (layer "F.Cu") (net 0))
 (segment (start 241.935 160.02) (end 229.87 147.955) (width 0.25) (layer "F.Cu") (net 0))
 (segment (start 227.965 94.615) (end 170.815 94.615) (width 0.25) (layer "F.Cu") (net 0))
 (segment (start 281.305 149.225) (end 281.305 130.81) (width 0.25) (layer "F.Cu") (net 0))
 (segment (start 275.59 200.66) (end 276.225 200.025) (width 0.25) (layer "F.Cu") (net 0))
 (segment (start 280.67 169.545) (end 281.305 168.91) (width 0.25) (layer "F.Cu") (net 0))
 (segment (start 175.895 160.02) (end 182.245 160.02) (width 0.25) (layer "F.Cu") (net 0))
 (segment (start 246.38 173.99) (end 259.08 186.69) (width 0.25) (layer "F.Cu") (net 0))
 (segment (start 165.735 116.205) (end 166.37 116.84) (width 0.25) (layer "F.Cu") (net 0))
 (segment (start 156.21 133.35) (end 156.21 128.905) (width 0.25) (layer "F.Cu") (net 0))
 (segment (start 277.495 127) (end 278.765 128.27) (width 0.25) (layer "F.Cu") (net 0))
 (segment (start 273.05 186.69) (end 280.035 193.675) (width 0.25) (layer "F.Cu") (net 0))
 (segment (start 219.71 201.93) (end 276.86 201.93) (width 0.25) (layer "F.Cu") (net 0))
 (segment (start 270.51 143.51) (end 269.875 143.51) (width 0.25) (layer "F.Cu") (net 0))
 (segment (start 167.64 173.99) (end 172.085 178.435) (width 0.25) (layer "F.Cu") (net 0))
 (segment (start 277.495 133.35) (end 277.495 140.335) (width 0.25) (layer "F.Cu") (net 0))
 (segment (start 170.18 133.35) (end 179.07 133.35) (width 0.25) (layer "F.Cu") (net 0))
 (segment (start 280.035 89.535) (end 278.13 89.535) (width 0.25) (layer "F.Cu") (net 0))
 (segment (start 176.53 105.41) (end 182.88 105.41) (width 0.25) (layer "F.Cu") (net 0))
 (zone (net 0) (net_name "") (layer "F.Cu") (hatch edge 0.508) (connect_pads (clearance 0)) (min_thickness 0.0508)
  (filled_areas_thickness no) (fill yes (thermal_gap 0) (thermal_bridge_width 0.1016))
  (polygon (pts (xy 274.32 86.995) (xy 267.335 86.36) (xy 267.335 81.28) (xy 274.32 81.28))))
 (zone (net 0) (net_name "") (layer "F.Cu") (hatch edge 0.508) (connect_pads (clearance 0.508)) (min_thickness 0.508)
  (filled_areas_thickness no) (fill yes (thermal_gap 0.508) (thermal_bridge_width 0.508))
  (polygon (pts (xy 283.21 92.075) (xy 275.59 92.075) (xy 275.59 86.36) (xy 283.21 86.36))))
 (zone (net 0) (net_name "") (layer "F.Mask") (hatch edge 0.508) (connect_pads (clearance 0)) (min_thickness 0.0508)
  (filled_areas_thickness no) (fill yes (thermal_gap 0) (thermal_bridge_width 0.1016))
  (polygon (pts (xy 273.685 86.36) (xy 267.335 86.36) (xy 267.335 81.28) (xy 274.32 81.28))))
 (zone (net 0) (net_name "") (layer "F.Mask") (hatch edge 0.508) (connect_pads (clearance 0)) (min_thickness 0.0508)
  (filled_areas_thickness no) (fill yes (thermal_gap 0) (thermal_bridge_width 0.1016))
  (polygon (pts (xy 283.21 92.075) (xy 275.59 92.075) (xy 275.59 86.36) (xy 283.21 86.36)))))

